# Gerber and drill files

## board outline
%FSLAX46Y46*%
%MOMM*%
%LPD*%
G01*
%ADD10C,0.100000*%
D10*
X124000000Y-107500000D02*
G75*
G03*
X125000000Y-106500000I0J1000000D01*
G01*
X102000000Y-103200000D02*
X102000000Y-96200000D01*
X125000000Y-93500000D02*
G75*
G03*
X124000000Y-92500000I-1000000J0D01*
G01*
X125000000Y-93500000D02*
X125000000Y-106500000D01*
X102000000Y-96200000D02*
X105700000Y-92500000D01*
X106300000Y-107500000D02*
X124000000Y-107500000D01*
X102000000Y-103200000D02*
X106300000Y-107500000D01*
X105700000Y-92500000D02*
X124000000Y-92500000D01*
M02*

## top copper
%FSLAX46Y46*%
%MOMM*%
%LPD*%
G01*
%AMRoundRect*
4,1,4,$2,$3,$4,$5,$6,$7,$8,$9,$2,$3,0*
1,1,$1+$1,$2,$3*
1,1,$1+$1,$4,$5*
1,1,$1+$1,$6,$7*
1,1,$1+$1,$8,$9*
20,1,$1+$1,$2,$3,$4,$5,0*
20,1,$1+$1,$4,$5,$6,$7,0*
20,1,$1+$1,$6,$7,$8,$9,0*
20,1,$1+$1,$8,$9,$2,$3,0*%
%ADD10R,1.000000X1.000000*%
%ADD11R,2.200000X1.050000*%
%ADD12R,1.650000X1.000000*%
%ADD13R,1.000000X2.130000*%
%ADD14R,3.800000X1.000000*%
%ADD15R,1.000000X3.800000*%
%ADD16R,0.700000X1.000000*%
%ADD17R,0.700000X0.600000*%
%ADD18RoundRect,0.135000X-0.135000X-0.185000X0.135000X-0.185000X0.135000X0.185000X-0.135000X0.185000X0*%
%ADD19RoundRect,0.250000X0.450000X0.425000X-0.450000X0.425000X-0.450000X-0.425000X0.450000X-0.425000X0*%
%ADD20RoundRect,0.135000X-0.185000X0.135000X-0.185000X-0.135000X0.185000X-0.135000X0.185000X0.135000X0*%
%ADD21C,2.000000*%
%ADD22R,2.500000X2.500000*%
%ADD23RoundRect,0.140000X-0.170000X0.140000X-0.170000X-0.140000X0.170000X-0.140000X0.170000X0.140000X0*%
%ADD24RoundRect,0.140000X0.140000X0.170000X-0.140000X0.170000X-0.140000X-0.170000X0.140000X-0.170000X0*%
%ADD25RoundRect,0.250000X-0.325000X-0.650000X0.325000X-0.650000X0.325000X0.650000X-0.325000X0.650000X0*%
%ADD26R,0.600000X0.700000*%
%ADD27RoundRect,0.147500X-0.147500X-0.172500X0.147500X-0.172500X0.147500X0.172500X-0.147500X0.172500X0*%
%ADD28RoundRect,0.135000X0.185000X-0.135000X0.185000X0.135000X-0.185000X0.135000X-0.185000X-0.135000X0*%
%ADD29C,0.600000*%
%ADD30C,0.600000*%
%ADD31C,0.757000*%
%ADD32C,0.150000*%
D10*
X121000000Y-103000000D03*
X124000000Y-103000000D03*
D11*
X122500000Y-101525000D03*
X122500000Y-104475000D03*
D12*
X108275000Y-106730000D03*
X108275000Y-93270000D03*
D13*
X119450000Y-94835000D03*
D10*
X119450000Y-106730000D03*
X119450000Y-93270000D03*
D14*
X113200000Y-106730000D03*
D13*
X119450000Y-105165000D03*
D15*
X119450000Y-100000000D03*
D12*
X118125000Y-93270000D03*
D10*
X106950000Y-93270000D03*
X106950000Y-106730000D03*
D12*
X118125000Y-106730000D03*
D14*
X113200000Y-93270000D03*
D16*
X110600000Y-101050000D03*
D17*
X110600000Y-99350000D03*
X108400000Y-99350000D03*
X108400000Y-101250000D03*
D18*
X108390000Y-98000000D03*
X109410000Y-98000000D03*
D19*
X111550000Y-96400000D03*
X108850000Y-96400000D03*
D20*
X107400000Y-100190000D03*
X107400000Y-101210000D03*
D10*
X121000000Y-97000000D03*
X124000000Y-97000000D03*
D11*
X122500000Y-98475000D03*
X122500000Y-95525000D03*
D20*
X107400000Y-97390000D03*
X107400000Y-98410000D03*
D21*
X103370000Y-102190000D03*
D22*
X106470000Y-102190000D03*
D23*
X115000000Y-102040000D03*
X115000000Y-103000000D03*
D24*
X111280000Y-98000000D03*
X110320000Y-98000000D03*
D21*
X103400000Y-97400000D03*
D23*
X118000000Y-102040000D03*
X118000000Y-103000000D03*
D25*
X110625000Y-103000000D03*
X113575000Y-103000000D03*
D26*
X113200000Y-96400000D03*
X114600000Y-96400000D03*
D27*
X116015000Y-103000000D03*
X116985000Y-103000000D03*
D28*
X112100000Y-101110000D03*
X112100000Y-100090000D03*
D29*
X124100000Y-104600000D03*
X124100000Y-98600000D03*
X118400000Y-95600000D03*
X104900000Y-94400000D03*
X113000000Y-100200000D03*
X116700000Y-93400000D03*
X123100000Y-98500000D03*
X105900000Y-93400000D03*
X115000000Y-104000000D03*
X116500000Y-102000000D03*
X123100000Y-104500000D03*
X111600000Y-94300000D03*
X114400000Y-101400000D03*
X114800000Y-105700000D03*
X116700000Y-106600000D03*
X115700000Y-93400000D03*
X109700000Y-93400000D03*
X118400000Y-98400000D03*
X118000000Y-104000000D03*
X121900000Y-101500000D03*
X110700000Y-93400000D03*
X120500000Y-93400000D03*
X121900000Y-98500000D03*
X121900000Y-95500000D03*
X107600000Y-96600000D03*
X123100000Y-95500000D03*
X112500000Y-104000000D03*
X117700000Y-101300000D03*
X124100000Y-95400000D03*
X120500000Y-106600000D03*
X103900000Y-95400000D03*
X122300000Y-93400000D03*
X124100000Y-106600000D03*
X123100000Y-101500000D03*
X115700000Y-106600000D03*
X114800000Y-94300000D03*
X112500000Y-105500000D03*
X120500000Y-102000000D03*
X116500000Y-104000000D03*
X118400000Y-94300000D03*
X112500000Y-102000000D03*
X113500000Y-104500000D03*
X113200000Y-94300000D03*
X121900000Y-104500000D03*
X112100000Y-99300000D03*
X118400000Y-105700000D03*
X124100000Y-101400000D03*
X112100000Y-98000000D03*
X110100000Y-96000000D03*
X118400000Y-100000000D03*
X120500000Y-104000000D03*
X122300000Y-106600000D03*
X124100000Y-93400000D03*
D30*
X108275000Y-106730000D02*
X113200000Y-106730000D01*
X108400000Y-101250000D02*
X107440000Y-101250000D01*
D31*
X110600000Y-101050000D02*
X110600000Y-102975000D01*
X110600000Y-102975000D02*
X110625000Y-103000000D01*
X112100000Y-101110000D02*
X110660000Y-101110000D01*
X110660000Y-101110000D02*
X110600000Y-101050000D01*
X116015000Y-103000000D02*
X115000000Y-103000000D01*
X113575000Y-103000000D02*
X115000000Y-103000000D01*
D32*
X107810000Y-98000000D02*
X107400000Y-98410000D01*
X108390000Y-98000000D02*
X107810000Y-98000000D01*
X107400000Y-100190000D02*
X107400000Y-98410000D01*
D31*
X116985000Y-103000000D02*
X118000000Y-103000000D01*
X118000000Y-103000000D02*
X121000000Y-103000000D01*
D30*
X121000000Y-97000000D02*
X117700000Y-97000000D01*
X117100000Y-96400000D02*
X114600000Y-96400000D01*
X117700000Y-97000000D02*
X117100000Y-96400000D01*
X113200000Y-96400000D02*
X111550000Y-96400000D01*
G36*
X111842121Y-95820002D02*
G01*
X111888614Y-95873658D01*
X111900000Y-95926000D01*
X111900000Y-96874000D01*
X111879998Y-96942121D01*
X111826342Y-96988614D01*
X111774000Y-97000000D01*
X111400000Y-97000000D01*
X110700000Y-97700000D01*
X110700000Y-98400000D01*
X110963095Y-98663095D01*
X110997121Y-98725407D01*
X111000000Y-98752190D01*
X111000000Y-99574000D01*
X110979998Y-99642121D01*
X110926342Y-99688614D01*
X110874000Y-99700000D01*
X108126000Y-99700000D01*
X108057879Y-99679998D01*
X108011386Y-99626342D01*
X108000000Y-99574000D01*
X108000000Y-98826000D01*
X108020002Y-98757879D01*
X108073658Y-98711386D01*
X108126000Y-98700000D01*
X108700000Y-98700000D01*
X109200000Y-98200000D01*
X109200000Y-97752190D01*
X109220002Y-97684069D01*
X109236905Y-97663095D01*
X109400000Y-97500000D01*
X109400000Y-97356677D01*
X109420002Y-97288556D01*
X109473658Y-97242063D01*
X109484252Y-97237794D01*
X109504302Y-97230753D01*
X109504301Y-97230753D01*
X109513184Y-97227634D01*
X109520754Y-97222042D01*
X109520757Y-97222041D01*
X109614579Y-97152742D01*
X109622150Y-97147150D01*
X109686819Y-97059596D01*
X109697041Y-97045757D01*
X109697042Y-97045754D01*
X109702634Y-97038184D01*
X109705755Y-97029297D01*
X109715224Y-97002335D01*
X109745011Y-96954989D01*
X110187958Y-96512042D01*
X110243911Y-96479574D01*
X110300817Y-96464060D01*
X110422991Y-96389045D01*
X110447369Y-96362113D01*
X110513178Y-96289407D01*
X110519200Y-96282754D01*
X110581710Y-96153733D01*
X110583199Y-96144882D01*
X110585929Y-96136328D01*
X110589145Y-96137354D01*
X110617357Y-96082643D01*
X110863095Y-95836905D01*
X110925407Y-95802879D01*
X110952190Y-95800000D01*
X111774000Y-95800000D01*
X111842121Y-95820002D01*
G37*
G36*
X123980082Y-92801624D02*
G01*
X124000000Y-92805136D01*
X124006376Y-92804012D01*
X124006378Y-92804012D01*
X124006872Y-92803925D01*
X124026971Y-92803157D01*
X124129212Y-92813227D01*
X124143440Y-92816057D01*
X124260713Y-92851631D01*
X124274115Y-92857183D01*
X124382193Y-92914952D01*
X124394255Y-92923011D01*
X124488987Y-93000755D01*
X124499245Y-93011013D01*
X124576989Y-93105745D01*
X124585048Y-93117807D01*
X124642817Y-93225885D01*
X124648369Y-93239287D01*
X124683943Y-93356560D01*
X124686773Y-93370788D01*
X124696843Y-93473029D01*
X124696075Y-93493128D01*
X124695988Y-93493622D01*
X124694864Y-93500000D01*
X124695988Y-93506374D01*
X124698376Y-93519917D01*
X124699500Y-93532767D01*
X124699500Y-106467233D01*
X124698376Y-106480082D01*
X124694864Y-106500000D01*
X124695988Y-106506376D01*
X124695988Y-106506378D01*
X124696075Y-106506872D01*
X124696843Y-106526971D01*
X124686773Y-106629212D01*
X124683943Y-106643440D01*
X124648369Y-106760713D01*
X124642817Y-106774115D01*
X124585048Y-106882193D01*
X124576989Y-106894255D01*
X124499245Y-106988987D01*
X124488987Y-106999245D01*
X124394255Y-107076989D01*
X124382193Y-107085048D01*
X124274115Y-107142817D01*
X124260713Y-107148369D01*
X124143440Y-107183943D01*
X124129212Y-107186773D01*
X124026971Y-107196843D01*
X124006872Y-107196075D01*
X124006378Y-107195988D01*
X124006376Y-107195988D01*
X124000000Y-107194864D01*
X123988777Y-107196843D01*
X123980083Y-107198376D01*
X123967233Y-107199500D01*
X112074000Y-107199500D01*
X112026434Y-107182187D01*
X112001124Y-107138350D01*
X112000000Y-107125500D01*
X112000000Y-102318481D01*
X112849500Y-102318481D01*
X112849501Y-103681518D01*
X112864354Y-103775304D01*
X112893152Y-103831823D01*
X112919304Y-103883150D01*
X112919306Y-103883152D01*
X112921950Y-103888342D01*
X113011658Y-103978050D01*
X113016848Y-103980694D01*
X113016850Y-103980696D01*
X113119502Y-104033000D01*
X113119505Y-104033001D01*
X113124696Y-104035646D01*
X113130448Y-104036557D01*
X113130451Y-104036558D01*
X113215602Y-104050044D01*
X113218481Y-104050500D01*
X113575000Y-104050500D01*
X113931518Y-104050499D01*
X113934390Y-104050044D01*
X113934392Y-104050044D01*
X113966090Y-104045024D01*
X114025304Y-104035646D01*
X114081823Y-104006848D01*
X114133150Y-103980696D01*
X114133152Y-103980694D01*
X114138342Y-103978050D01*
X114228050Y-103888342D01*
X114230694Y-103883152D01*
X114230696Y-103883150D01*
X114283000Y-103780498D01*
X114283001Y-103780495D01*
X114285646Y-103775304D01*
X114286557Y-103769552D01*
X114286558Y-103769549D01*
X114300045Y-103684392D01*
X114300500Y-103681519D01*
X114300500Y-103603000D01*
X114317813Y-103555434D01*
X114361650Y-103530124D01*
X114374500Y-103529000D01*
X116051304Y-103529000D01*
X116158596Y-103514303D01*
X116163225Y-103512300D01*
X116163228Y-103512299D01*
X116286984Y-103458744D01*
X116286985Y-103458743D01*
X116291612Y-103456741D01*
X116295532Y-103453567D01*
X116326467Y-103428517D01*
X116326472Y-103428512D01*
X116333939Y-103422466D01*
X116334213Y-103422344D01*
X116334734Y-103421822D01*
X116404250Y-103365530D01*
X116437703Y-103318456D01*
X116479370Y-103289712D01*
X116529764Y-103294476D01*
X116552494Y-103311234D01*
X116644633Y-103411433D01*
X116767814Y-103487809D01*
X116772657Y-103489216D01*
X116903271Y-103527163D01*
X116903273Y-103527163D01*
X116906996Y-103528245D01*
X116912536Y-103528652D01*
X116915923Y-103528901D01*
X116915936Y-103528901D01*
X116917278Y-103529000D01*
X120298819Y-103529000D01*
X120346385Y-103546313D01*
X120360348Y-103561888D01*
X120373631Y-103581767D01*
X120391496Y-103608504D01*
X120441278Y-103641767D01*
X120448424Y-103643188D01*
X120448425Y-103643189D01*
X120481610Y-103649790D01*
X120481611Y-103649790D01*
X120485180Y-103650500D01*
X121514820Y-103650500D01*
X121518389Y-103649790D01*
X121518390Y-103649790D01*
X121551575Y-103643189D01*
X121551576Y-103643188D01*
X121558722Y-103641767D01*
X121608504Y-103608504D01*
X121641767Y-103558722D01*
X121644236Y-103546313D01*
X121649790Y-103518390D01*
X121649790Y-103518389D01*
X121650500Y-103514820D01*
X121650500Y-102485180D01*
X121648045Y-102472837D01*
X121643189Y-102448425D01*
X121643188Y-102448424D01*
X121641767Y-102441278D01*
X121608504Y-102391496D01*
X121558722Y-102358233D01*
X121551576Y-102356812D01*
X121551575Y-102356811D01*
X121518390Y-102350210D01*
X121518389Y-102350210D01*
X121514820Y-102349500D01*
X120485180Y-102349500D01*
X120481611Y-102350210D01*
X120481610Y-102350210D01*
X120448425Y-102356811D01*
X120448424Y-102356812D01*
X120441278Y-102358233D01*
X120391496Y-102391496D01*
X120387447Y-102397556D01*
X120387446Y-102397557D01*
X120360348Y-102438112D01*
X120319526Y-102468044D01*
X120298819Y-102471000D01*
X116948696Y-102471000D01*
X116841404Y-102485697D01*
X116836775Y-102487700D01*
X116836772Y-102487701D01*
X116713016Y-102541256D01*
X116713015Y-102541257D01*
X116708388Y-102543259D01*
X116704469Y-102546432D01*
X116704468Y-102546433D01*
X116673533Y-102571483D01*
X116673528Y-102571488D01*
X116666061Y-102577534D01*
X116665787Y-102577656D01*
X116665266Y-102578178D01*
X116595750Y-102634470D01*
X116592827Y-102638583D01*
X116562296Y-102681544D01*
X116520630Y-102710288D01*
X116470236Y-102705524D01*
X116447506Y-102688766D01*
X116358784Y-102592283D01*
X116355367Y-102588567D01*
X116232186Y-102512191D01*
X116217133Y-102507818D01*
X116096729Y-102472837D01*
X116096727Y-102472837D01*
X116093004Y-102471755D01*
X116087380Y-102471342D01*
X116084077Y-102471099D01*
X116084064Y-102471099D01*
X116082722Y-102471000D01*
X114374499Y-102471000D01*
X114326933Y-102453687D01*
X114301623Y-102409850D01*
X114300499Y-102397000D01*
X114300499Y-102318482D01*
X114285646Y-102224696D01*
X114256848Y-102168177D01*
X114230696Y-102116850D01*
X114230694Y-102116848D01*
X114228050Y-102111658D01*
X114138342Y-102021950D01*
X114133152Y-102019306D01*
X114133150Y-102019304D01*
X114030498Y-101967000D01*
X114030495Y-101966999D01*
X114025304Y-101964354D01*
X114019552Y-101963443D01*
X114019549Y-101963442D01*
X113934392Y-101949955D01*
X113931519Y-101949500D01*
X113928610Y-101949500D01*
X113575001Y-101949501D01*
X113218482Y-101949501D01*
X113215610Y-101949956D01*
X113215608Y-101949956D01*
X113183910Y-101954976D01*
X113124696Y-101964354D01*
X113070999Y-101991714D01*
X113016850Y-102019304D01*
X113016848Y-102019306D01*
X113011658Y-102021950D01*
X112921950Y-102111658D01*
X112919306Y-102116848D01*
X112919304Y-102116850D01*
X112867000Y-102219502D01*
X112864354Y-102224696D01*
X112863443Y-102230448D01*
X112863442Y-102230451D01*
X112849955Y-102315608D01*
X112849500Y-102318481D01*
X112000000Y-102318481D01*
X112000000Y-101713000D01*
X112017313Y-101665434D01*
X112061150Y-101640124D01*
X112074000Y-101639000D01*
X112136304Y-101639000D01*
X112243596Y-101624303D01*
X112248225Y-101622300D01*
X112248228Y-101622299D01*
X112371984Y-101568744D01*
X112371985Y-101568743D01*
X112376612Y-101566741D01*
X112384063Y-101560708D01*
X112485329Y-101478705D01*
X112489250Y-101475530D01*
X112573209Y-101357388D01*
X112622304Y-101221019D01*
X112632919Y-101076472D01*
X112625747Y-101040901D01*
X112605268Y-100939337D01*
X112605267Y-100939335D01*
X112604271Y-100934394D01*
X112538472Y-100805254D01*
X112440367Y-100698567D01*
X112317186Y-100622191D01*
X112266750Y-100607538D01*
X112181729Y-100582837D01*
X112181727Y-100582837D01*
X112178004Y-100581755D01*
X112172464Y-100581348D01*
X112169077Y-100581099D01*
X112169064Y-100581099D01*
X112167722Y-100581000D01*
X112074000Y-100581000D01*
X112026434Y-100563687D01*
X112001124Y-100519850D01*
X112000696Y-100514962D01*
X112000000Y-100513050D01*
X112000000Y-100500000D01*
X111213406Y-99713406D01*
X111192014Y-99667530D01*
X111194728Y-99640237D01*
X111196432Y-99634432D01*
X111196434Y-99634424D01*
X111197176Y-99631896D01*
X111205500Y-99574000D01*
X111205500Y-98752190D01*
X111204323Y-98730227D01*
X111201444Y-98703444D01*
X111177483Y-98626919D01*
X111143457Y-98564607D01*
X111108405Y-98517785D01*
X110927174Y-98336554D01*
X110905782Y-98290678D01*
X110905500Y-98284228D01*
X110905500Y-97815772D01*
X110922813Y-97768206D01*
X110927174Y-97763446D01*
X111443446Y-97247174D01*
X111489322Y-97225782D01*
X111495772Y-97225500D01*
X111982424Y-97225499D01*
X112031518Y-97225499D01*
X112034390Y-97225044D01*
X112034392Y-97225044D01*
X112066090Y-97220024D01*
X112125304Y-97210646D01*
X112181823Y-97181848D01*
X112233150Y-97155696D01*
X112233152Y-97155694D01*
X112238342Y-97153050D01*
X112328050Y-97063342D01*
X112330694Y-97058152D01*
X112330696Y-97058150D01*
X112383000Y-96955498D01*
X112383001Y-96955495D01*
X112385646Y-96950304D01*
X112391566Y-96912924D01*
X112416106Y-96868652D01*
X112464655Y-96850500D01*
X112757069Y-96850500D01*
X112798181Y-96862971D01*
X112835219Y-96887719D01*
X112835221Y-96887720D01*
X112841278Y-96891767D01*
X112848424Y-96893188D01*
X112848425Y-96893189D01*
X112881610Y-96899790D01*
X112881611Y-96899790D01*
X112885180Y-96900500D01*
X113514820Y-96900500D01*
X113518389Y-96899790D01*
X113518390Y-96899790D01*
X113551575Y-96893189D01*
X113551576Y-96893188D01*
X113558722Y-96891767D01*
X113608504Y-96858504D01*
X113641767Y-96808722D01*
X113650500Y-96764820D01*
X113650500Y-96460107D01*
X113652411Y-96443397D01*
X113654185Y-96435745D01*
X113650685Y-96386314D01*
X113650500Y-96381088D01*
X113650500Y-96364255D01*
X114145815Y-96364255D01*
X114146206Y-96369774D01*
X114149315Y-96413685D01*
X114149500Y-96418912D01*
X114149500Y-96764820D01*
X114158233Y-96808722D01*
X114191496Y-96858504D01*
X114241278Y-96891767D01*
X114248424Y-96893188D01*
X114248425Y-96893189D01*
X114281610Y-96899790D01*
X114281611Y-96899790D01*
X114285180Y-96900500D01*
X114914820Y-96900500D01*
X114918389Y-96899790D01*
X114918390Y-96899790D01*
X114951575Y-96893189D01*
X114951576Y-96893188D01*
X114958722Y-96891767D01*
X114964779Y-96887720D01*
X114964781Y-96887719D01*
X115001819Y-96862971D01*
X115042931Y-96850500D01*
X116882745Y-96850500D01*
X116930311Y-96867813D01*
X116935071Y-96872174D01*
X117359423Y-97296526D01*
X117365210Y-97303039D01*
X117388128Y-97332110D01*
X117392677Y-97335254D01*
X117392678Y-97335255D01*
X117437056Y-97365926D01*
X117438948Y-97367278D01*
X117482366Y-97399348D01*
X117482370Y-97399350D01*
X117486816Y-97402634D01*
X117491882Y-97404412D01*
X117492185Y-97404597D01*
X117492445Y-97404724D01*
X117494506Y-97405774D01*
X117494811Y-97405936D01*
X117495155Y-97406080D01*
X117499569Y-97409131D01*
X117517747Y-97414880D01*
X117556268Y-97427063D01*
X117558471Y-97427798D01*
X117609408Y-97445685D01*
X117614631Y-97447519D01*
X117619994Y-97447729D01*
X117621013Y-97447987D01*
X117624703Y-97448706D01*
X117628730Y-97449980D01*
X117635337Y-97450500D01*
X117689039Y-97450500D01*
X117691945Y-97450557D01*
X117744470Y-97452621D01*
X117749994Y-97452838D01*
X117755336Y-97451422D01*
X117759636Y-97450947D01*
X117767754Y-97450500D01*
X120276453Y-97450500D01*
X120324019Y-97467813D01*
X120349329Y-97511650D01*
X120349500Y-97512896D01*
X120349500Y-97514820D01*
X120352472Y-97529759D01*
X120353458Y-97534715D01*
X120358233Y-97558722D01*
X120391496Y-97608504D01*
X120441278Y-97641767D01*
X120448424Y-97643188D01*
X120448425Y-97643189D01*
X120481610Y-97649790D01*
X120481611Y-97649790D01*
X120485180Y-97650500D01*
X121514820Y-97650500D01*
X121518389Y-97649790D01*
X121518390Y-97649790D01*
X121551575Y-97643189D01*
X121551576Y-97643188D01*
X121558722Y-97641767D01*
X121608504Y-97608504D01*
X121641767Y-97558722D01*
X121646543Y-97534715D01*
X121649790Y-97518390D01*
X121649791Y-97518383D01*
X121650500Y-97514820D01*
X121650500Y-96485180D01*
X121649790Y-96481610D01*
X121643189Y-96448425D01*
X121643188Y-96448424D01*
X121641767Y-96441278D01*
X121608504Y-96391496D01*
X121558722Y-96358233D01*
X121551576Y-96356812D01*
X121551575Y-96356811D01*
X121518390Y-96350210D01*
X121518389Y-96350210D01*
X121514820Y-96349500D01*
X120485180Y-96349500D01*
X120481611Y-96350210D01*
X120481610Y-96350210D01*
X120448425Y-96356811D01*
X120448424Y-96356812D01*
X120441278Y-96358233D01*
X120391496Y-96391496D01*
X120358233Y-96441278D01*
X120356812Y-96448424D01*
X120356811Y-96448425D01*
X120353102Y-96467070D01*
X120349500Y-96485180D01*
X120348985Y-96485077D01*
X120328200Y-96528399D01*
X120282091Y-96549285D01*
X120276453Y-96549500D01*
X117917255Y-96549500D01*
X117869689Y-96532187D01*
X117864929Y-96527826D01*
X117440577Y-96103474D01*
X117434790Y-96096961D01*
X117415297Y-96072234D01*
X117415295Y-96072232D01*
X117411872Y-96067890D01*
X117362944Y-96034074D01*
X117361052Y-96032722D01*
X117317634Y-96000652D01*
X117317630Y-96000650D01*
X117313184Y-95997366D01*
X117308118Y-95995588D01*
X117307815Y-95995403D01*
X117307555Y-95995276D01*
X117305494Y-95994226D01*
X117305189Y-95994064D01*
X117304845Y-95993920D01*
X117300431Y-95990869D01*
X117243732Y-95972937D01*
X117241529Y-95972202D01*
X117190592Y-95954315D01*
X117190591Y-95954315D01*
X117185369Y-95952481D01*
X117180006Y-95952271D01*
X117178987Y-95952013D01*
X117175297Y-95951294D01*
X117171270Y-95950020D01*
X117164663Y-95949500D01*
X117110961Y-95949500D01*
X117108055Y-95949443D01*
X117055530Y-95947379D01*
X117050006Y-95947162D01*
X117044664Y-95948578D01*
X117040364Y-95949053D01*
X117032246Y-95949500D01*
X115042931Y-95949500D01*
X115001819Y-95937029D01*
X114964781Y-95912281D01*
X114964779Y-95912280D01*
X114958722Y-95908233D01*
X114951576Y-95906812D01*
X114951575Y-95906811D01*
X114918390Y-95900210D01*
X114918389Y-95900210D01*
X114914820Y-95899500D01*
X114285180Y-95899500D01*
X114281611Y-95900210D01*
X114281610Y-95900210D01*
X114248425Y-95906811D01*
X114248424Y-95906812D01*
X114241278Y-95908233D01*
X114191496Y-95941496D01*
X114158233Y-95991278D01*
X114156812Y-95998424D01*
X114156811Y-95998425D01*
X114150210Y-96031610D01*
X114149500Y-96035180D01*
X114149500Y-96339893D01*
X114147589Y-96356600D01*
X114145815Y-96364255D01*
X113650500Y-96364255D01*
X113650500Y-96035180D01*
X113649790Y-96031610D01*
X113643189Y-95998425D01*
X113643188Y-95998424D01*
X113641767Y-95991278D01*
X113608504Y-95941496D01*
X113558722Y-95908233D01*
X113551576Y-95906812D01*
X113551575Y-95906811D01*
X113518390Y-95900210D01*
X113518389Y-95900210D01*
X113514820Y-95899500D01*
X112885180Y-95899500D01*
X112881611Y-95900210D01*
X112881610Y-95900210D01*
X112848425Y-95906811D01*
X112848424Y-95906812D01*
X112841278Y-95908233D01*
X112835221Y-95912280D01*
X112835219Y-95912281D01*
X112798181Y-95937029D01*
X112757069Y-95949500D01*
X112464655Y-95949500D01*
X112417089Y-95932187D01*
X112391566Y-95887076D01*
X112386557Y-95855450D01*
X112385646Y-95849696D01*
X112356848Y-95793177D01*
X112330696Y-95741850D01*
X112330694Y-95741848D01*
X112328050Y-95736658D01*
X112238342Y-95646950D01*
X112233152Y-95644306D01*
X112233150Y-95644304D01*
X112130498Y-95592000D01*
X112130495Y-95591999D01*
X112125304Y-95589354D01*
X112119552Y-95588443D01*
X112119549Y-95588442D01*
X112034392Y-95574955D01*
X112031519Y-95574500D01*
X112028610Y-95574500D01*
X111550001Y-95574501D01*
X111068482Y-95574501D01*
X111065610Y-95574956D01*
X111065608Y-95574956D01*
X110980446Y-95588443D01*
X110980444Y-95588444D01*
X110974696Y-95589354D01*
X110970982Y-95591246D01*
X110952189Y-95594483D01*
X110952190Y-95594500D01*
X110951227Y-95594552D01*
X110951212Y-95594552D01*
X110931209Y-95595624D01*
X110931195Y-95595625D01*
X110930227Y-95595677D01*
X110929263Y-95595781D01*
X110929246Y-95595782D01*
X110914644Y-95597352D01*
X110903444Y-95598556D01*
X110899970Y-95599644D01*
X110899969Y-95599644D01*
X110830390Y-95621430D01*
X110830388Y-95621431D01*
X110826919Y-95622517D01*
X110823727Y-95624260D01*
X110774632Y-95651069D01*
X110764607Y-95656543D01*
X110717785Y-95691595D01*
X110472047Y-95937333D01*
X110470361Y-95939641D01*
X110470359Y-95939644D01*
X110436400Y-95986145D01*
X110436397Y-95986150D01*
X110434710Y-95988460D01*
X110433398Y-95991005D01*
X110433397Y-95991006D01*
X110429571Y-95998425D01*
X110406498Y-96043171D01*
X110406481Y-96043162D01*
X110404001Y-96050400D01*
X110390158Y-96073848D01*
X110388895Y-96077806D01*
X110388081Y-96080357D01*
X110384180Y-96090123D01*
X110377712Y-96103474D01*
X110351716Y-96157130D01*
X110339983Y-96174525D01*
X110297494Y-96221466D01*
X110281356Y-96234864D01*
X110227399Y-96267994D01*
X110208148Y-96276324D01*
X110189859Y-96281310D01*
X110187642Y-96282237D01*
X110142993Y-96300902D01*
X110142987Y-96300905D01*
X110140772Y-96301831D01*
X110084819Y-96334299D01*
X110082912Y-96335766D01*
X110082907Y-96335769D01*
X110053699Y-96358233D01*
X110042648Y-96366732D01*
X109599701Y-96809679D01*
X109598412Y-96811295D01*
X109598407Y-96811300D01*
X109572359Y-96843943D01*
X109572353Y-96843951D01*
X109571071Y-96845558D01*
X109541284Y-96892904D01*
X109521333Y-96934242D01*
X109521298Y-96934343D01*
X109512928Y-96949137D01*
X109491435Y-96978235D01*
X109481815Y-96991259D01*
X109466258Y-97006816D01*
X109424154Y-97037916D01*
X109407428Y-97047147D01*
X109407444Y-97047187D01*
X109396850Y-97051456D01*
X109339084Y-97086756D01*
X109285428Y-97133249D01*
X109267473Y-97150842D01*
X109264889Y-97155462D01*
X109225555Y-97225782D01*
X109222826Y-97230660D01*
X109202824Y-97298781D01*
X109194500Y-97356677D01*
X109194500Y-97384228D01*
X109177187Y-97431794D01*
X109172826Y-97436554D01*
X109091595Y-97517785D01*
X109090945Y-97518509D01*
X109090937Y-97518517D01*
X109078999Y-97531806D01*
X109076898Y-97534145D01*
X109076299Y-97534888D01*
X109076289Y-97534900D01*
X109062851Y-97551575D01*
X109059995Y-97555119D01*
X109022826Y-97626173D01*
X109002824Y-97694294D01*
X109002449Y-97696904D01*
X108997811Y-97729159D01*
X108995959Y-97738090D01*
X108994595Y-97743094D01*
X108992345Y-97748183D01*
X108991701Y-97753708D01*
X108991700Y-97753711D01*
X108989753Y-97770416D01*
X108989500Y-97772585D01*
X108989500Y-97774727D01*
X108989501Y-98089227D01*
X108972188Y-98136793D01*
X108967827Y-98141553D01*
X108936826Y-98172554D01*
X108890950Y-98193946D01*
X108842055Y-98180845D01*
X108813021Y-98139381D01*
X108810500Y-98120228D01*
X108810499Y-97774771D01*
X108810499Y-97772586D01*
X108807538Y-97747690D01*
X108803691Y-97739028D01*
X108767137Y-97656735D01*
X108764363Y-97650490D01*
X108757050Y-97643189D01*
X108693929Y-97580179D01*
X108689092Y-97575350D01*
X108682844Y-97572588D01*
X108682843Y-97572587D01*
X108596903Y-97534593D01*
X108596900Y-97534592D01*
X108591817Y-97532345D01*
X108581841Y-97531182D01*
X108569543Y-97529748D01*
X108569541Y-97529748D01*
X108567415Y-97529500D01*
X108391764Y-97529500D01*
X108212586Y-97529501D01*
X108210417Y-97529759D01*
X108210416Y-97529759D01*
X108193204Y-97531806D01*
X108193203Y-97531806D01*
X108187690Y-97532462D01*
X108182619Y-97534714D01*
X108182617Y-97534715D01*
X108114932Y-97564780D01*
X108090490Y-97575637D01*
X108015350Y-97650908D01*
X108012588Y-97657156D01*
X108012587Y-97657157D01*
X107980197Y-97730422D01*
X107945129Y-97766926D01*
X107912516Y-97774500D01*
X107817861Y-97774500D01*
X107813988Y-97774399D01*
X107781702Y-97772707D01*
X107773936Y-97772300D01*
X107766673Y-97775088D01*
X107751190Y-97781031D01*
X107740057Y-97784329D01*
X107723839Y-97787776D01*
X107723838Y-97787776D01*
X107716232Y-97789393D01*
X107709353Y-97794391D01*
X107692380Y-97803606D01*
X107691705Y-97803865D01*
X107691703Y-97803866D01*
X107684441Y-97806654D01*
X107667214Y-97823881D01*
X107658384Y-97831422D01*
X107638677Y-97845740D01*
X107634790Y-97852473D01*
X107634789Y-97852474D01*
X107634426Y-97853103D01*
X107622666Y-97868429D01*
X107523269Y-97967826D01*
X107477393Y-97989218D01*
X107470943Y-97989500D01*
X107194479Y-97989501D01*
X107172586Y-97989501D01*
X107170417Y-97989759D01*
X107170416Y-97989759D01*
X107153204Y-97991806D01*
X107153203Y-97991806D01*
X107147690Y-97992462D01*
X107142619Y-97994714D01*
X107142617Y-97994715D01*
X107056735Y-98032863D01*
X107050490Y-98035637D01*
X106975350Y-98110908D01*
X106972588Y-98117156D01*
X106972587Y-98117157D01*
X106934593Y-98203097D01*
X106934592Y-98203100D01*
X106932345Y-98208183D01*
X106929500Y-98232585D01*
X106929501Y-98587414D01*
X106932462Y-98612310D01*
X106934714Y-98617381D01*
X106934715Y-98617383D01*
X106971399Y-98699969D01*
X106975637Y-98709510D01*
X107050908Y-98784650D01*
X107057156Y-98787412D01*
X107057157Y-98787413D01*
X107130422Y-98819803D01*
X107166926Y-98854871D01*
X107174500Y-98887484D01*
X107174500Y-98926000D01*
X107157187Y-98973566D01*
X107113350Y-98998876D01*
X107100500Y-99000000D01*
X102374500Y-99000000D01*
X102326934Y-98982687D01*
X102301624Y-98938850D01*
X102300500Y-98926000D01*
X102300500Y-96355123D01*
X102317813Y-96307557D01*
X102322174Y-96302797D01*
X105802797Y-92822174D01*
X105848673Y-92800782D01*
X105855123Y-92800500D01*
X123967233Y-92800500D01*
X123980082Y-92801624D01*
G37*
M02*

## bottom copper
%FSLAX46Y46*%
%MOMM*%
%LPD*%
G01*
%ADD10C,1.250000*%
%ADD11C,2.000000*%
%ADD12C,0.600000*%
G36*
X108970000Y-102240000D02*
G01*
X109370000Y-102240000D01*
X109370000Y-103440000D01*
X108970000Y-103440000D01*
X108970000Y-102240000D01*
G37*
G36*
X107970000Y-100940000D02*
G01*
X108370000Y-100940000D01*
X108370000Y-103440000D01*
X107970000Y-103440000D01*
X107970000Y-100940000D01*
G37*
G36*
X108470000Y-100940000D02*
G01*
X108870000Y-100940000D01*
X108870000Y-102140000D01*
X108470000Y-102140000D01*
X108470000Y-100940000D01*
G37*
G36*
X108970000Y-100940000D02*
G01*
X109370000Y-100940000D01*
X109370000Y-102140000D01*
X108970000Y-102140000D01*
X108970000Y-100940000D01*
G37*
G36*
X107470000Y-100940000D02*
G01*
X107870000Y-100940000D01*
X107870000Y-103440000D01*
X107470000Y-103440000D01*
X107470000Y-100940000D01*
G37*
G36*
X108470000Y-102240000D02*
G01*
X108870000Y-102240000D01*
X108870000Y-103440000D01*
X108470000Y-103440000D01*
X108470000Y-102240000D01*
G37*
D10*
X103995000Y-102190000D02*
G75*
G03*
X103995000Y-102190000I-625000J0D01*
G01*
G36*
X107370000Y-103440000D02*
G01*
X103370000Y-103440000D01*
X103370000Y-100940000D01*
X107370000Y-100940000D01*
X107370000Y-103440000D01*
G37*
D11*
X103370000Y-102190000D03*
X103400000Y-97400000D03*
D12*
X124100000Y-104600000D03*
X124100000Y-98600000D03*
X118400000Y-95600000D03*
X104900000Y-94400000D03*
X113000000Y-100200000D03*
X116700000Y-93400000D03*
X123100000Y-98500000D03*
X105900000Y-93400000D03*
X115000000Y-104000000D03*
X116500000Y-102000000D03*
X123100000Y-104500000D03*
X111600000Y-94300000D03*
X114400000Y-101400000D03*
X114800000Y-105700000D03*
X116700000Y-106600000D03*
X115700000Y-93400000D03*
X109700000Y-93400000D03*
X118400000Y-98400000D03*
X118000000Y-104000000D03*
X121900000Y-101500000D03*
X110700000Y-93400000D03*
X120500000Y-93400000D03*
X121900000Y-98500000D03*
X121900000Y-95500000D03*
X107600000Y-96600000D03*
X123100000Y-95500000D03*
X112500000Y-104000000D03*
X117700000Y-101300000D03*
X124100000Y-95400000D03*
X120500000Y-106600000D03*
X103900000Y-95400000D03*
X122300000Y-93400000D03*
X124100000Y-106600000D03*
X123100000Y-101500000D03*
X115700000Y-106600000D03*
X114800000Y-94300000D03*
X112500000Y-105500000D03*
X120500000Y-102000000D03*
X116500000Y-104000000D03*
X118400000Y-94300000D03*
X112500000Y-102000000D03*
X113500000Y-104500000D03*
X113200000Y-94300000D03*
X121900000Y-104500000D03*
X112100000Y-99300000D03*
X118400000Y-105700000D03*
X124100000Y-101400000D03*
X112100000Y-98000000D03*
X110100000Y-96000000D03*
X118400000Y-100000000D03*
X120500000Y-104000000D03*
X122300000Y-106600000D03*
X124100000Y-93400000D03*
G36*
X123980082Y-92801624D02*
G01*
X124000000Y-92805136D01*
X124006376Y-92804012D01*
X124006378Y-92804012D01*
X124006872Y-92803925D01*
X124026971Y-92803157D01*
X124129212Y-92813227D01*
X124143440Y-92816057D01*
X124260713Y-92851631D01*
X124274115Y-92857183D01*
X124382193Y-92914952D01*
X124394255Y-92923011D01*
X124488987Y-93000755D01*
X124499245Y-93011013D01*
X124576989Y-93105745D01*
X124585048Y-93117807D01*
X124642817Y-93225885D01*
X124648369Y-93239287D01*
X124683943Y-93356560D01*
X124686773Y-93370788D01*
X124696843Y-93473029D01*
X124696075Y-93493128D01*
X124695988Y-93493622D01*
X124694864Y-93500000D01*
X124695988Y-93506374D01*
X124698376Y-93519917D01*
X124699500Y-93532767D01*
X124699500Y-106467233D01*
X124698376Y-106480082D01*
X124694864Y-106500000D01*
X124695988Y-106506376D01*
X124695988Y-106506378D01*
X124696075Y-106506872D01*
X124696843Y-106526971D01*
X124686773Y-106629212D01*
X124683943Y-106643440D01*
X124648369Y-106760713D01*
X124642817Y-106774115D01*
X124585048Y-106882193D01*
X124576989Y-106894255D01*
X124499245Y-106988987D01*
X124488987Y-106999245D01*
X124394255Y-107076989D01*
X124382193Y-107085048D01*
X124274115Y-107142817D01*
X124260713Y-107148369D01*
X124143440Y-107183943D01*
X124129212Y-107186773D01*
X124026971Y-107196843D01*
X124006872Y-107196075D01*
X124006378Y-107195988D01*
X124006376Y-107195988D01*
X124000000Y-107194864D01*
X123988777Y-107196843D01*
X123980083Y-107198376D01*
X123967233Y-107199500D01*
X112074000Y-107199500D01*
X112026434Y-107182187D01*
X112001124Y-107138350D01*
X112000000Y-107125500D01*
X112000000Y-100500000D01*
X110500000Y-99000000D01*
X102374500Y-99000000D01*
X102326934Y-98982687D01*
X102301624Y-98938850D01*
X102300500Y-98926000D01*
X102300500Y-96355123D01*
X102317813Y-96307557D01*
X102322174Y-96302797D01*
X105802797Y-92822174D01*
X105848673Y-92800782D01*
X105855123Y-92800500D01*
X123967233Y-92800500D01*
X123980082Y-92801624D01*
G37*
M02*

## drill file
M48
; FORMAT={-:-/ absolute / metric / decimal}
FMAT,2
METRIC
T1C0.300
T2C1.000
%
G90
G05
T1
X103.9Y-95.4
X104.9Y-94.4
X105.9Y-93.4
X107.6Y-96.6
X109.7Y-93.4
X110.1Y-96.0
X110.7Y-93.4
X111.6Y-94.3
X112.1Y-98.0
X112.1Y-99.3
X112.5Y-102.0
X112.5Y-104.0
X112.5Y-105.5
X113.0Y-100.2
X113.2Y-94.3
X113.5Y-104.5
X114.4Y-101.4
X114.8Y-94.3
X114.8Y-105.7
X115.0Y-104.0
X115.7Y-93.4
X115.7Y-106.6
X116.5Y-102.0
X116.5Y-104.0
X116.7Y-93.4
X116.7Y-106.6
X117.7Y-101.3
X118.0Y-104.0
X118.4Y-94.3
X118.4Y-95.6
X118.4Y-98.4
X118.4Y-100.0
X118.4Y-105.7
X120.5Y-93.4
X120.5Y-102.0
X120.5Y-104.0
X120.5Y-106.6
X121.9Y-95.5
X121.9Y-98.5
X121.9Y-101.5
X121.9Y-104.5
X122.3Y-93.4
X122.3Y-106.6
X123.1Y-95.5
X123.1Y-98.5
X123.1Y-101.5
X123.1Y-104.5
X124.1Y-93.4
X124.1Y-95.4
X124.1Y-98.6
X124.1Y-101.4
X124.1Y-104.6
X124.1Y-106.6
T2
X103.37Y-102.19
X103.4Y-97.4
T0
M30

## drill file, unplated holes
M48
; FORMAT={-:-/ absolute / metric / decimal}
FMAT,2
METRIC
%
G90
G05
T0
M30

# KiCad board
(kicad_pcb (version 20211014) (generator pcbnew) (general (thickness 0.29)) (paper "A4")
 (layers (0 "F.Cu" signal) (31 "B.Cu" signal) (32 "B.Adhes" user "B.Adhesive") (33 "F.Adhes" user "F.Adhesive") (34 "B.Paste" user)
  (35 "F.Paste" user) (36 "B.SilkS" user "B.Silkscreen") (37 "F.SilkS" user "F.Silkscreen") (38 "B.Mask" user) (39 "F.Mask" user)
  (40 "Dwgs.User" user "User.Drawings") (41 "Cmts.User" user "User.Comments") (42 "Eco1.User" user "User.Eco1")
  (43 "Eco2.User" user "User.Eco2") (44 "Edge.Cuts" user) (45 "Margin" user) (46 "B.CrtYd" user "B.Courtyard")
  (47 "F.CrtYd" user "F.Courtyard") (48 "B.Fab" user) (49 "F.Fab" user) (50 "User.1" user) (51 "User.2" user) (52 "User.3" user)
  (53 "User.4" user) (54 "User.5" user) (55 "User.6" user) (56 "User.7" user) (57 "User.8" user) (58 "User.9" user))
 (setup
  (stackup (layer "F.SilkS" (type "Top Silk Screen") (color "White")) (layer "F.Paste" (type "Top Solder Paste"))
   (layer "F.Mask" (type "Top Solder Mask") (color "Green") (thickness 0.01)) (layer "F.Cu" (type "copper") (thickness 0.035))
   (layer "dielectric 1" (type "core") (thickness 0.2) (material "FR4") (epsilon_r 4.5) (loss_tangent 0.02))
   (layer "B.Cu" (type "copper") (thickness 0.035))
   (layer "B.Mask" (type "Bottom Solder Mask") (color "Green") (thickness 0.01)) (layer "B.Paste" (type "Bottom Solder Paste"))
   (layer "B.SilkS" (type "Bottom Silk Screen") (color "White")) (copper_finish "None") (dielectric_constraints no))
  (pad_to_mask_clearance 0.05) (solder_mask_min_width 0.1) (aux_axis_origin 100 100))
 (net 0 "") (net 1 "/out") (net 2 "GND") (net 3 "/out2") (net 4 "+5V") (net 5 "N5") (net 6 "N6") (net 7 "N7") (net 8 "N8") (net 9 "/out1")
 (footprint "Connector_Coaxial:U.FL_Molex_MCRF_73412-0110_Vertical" (layer "F.Cu") (at 122.5 103 -90)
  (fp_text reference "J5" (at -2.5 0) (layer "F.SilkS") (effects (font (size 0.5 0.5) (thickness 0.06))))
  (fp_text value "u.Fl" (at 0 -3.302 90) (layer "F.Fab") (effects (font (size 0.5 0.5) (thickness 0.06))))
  (pad "1" smd rect (at 0 1.5 270) (size 1 1) (layers "F.Cu" "F.Paste" "F.Mask") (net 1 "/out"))
  (pad "2" smd rect (at 0 -1.5 270) (size 1 1) (layers "F.Cu" "F.Paste" "F.Mask") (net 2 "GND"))
  (pad "2" smd rect (at -1.475 0 270) (size 1.05 2.2) (layers "F.Cu" "F.Paste" "F.Mask") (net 2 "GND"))
  (pad "2" smd rect (at 1.475 0 270) (size 1.05 2.2) (layers "F.Cu" "F.Paste" "F.Mask") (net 2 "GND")))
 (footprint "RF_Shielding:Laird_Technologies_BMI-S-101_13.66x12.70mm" (layer "F.Cu") (at 113.2 100) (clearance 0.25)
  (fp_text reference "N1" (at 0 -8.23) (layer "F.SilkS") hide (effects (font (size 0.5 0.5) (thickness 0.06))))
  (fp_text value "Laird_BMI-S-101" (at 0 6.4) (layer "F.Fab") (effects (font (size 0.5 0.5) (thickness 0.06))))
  (pad "1" smd rect (at -4.925 6.73) (size 1.65 1) (layers "F.Cu" "F.Paste" "F.Mask") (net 2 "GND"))
  (pad "1" smd rect (at -4.925 -6.73) (size 1.65 1) (layers "F.Cu" "F.Paste" "F.Mask") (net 2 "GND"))
  (pad "1" smd rect (at 6.25 -5.165) (size 1 2.13) (layers "F.Cu" "F.Paste" "F.Mask") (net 2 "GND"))
  (pad "1" smd rect (at 6.25 6.73) (size 1 1) (layers "F.Cu" "F.Paste" "F.Mask") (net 2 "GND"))
  (pad "1" smd rect (at 6.25 -6.73) (size 1 1) (layers "F.Cu" "F.Paste" "F.Mask") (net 2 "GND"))
  (pad "1" smd rect (at 0 6.73) (size 3.8 1) (layers "F.Cu" "F.Paste" "F.Mask") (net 2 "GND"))
  (pad "1" smd rect (at 6.25 5.165) (size 1 2.13) (layers "F.Cu" "F.Paste" "F.Mask") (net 2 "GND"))
  (pad "1" smd rect (at 6.25 0) (size 1 3.8) (layers "F.Cu" "F.Paste" "F.Mask") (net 2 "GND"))
  (pad "1" smd rect (at 4.925 -6.73) (size 1.65 1) (layers "F.Cu" "F.Paste" "F.Mask") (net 2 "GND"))
  (pad "1" smd rect (at -6.25 -6.73) (size 1 1) (layers "F.Cu" "F.Paste" "F.Mask") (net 2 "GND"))
  (pad "1" smd rect (at -6.25 6.73) (size 1 1) (layers "F.Cu" "F.Paste" "F.Mask") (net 2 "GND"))
  (pad "1" smd rect (at 4.925 6.73) (size 1.65 1) (layers "F.Cu" "F.Paste" "F.Mask") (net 2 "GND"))
  (pad "1" smd rect (at 0 -6.73) (size 3.8 1) (layers "F.Cu" "F.Paste" "F.Mask") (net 2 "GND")))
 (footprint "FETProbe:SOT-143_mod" (layer "F.Cu") (at 109.5 100.3 180)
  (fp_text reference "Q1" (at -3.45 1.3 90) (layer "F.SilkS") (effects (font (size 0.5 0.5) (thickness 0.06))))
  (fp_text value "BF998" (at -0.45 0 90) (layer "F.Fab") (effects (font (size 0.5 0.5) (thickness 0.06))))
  (pad "1" smd rect (at -1.1 -0.75 180) (size 0.7 1) (layers "F.Cu" "F.Paste" "F.Mask") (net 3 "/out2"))
  (pad "2" smd rect (at -1.1 0.95 180) (size 0.7 0.6) (layers "F.Cu" "F.Paste" "F.Mask") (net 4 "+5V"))
  (pad "3" smd rect (at 1.1 0.95 180) (size 0.7 0.6) (layers "F.Cu" "F.Paste" "F.Mask") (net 4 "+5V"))
  (pad "4" smd rect (at 1.1 -0.95 180) (size 0.7 0.6) (layers "F.Cu" "F.Paste" "F.Mask") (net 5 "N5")))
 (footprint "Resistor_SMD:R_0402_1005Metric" (layer "F.Cu") (at 108.9 98)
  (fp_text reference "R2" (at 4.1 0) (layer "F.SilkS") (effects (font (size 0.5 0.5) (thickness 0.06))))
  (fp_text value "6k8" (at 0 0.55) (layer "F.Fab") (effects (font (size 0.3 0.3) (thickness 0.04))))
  (pad "1" smd roundrect (at -0.51 0) (size 0.54 0.64) (layers "F.Cu" "F.Paste" "F.Mask") (roundrect_rratio 0.25) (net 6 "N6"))
  (pad "2" smd roundrect (at 0.51 0) (size 0.54 0.64) (layers "F.Cu" "F.Paste" "F.Mask") (roundrect_rratio 0.25) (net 4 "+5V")))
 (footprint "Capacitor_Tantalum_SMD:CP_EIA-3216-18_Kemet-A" (layer "F.Cu") (at 110.2 96.4 180)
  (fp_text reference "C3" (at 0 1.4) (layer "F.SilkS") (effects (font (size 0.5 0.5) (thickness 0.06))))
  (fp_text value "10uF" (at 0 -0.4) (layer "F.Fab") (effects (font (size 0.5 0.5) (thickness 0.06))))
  (pad "1" smd roundrect (at -1.35 0 180) (size 1.4 1.35) (layers "F.Cu" "F.Paste" "F.Mask") (roundrect_rratio 0.1851851852) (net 4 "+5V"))
  (pad "2" smd roundrect (at 1.35 0 180) (size 1.4 1.35) (layers "F.Cu" "F.Paste" "F.Mask") (roundrect_rratio 0.1851851852) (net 2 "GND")))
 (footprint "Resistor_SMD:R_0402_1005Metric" (layer "F.Cu") (at 107.4 100.7 -90)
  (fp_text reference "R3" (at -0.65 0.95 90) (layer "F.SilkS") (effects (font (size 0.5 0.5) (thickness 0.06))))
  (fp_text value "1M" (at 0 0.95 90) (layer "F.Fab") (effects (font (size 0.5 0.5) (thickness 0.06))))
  (pad "1" smd roundrect (at -0.51 0 270) (size 0.54 0.64) (layers "F.Cu" "F.Paste" "F.Mask") (roundrect_rratio 0.25) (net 6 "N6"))
  (pad "2" smd roundrect (at 0.51 0 270) (size 0.54 0.64) (layers "F.Cu" "F.Paste" "F.Mask") (roundrect_rratio 0.25) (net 5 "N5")))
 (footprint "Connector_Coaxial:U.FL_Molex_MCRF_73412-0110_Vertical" (layer "F.Cu") (at 122.5 97 -90)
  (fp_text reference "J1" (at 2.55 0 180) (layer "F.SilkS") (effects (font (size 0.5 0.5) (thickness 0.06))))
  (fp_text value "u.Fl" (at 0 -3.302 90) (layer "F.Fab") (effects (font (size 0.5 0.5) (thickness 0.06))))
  (pad "1" smd rect (at 0 1.5 270) (size 1 1) (layers "F.Cu" "F.Paste" "F.Mask") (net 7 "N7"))
  (pad "2" smd rect (at 0 -1.5 270) (size 1 1) (layers "F.Cu" "F.Paste" "F.Mask") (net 2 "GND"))
  (pad "2" smd rect (at 1.475 0 270) (size 1.05 2.2) (layers "F.Cu" "F.Paste" "F.Mask") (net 2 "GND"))
  (pad "2" smd rect (at -1.475 0 270) (size 1.05 2.2) (layers "F.Cu" "F.Paste" "F.Mask") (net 2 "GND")))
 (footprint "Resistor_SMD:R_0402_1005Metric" (layer "F.Cu") (at 107.4 97.9 -90)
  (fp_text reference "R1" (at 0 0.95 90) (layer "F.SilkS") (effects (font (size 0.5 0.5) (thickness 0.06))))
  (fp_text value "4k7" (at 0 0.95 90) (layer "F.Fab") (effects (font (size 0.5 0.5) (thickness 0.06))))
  (pad "1" smd roundrect (at -0.51 0 270) (size 0.54 0.64) (layers "F.Cu" "F.Paste" "F.Mask") (roundrect_rratio 0.25) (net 2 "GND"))
  (pad "2" smd roundrect (at 0.51 0 270) (size 0.54 0.64) (layers "F.Cu" "F.Paste" "F.Mask") (roundrect_rratio 0.25) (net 6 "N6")))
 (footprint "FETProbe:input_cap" (layer "F.Cu") (at 108.07 102.19)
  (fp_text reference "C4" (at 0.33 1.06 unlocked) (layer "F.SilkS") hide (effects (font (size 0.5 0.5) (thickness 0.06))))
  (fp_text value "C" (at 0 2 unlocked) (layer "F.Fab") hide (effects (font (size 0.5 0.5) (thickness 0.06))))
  (fp_rect (start 0.9 0.05) (end 1.3 1.25) (layer "B.Cu") (width 0) (fill solid))
  (fp_rect (start -0.1 -1.25) (end 0.3 1.25) (layer "B.Cu") (width 0) (fill solid))
  (fp_rect (start 0.4 -1.25) (end 0.8 -0.05) (layer "B.Cu") (width 0) (fill solid))
  (fp_rect (start 0.9 -1.25) (end 1.3 -0.05) (layer "B.Cu") (width 0) (fill solid))
  (fp_rect (start -0.6 -1.25) (end -0.2 1.25) (layer "B.Cu") (width 0) (fill solid))
  (fp_rect (start 0.4 0.05) (end 0.8 1.25) (layer "B.Cu") (width 0) (fill solid))
  (fp_circle (center -4.7 0) (end -3.45 0) (layer "B.Cu") (width 0) (fill solid))
  (fp_poly (pts (xy -4.7 -1.25) (xy -0.7 -1.25) (xy -0.7 1.25) (xy -4.7 1.25)) (layer "B.Cu") (width 0) (fill solid))
  (pad "1" thru_hole circle (at -4.7 0) (size 2 2) (drill 1) (layers *.Cu *.Mask) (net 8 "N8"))
  (pad "2" smd rect (at -1.6 0) (size 2.5 2.5) (layers "F.Cu") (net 5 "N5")))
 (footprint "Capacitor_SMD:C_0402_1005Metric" (layer "F.Cu") (at 115 102.52 -90)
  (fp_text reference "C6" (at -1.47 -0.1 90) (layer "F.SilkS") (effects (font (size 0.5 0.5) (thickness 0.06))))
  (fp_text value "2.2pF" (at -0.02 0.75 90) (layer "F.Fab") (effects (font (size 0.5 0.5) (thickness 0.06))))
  (pad "1" smd roundrect (at -0.48 0 270) (size 0.56 0.62) (layers "F.Cu" "F.Paste" "F.Mask") (roundrect_rratio 0.25) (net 2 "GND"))
  (pad "2" smd roundrect (at 0.48 0 270) (size 0.56 0.62) (layers "F.Cu" "F.Paste" "F.Mask") (roundrect_rratio 0.25) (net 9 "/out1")))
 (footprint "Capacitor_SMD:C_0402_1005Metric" (layer "F.Cu") (at 110.8 98 180)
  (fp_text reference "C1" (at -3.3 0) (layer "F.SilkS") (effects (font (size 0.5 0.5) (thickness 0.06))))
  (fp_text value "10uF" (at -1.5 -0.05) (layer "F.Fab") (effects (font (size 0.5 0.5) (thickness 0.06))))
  (pad "1" smd roundrect (at -0.48 0 180) (size 0.56 0.62) (layers "F.Cu" "F.Paste" "F.Mask") (roundrect_rratio 0.25) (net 2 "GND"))
  (pad "2" smd roundrect (at 0.48 0 180) (size 0.56 0.62) (layers "F.Cu" "F.Paste" "F.Mask") (roundrect_rratio 0.25) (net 4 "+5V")))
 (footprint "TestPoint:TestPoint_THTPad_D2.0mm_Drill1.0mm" (layer "F.Cu") (at 103.4 97.4)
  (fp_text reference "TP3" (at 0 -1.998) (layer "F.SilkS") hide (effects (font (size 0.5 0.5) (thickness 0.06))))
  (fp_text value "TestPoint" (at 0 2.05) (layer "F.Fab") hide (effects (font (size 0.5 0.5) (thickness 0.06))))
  (pad "1" thru_hole circle (at 0 0) (size 2 2) (drill 1) (layers *.Cu *.Mask) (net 2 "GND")))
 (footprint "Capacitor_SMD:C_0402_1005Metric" (layer "F.Cu") (at 118 102.52 -90)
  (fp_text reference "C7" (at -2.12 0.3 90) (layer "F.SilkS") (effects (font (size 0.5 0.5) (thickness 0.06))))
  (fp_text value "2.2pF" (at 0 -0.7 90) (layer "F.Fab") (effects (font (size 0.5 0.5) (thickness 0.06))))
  (pad "1" smd roundrect (at -0.48 0 270) (size 0.56 0.62) (layers "F.Cu" "F.Paste" "F.Mask") (roundrect_rratio 0.25) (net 2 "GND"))
  (pad "2" smd roundrect (at 0.48 0 270) (size 0.56 0.62) (layers "F.Cu" "F.Paste" "F.Mask") (roundrect_rratio 0.25) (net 1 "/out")))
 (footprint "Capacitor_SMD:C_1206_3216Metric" (layer "F.Cu") (at 112.1 103)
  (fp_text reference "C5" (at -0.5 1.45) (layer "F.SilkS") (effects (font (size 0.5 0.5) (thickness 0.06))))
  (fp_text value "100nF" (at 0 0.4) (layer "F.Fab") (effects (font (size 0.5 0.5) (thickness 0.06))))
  (pad "1" smd roundrect (at -1.475 0) (size 1.15 1.8) (layers "F.Cu" "F.Paste" "F.Mask") (roundrect_rratio 0.2173913043) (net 3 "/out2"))
  (pad "2" smd roundrect (at 1.475 0) (size 1.15 1.8) (layers "F.Cu" "F.Paste" "F.Mask") (roundrect_rratio 0.2173913043) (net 9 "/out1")))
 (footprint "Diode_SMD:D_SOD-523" (layer "F.Cu") (at 113.9 96.4)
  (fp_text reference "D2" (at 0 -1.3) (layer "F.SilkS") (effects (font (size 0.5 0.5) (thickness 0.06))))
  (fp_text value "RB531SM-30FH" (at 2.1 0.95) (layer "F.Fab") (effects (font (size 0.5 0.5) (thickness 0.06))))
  (pad "1" smd rect (at -0.7 0 180) (size 0.6 0.7) (layers "F.Cu" "F.Paste" "F.Mask") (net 4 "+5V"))
  (pad "2" smd rect (at 0.7 0 180) (size 0.6 0.7) (layers "F.Cu" "F.Paste" "F.Mask") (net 7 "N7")))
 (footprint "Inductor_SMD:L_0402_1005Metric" (layer "F.Cu") (at 116.5 103)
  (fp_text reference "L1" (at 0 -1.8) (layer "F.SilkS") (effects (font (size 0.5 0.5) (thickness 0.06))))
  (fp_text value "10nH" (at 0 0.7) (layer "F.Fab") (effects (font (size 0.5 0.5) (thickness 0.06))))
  (pad "1" smd roundrect (at -0.485 0) (size 0.59 0.64) (layers "F.Cu" "F.Paste" "F.Mask") (roundrect_rratio 0.25) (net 9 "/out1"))
  (pad "2" smd roundrect (at 0.485 0) (size 0.59 0.64) (layers "F.Cu" "F.Paste" "F.Mask") (roundrect_rratio 0.25) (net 1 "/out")))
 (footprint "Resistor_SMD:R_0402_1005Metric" (layer "F.Cu") (at 112.1 100.6 90)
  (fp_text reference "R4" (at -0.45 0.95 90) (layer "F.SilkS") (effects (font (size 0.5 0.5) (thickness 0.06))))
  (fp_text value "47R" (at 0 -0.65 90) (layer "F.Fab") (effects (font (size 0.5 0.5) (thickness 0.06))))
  (pad "1" smd roundrect (at -0.51 0 90) (size 0.54 0.64) (layers "F.Cu" "F.Paste" "F.Mask") (roundrect_rratio 0.25) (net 3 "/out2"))
  (pad "2" smd roundrect (at 0.51 0 90) (size 0.54 0.64) (layers "F.Cu" "F.Paste" "F.Mask") (roundrect_rratio 0.25) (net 2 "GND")))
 (gr_arc (start 125 106.5) (mid 124.707107 107.207107) (end 124 107.5) (layer "Edge.Cuts") (width 0.1))
 (gr_line (start 102 103.2) (end 102 96.2) (layer "Edge.Cuts") (width 0.1))
 (gr_arc (start 124 92.5) (mid 124.707107 92.792893) (end 125 93.5) (layer "Edge.Cuts") (width 0.1))
 (gr_line (start 125 93.5) (end 125 106.5) (layer "Edge.Cuts") (width 0.1))
 (gr_line (start 102 96.2) (end 105.7 92.5) (layer "Edge.Cuts") (width 0.1))
 (gr_line (start 106.3 107.5) (end 124 107.5) (layer "Edge.Cuts") (width 0.1))
 (gr_line (start 102 103.2) (end 106.3 107.5) (layer "Edge.Cuts") (width 0.1))
 (gr_line (start 105.7 92.5) (end 124 92.5) (layer "Edge.Cuts") (width 0.1))
 (segment (start 108.275 106.73) (end 113.2 106.73) (width 0.6) (layer "F.Cu") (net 2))
 (via (at 124.1 104.6) (size 0.6) (drill 0.3) (layers "F.Cu" "B.Cu") (free) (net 2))
 (via (at 124.1 98.6) (size 0.6) (drill 0.3) (layers "F.Cu" "B.Cu") (free) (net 2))
 (via (at 118.4 95.6) (size 0.6) (drill 0.3) (layers "F.Cu" "B.Cu") (free) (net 2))
 (via (at 104.9 94.4) (size 0.6) (drill 0.3) (layers "F.Cu" "B.Cu") (free) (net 2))
 (via (at 113 100.2) (size 0.6) (drill 0.3) (layers "F.Cu" "B.Cu") (free) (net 2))
 (via (at 116.7 93.4) (size 0.6) (drill 0.3) (layers "F.Cu" "B.Cu") (free) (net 2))
 (via (at 123.1 98.5) (size 0.6) (drill 0.3) (layers "F.Cu" "B.Cu") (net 2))
 (via (at 105.9 93.4) (size 0.6) (drill 0.3) (layers "F.Cu" "B.Cu") (free) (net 2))
 (via (at 115 104) (size 0.6) (drill 0.3) (layers "F.Cu" "B.Cu") (free) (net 2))
 (via (at 116.5 102) (size 0.6) (drill 0.3) (layers "F.Cu" "B.Cu") (free) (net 2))
 (via (at 123.1 104.5) (size 0.6) (drill 0.3) (layers "F.Cu" "B.Cu") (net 2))
 (via (at 111.6 94.3) (size 0.6) (drill 0.3) (layers "F.Cu" "B.Cu") (free) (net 2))
 (via (at 114.4 101.4) (size 0.6) (drill 0.3) (layers "F.Cu" "B.Cu") (free) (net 2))
 (via (at 114.8 105.7) (size 0.6) (drill 0.3) (layers "F.Cu" "B.Cu") (free) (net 2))
 (via (at 116.7 106.6) (size 0.6) (drill 0.3) (layers "F.Cu" "B.Cu") (free) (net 2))
 (via (at 115.7 93.4) (size 0.6) (drill 0.3) (layers "F.Cu" "B.Cu") (free) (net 2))
 (via (at 109.7 93.4) (size 0.6) (drill 0.3) (layers "F.Cu" "B.Cu") (free) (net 2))
 (via (at 118.4 98.4) (size 0.6) (drill 0.3) (layers "F.Cu" "B.Cu") (free) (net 2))
 (via (at 118 104) (size 0.6) (drill 0.3) (layers "F.Cu" "B.Cu") (free) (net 2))
 (via (at 121.9 101.5) (size 0.6) (drill 0.3) (layers "F.Cu" "B.Cu") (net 2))
 (via (at 110.7 93.4) (size 0.6) (drill 0.3) (layers "F.Cu" "B.Cu") (free) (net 2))
 (via (at 120.5 93.4) (size 0.6) (drill 0.3) (layers "F.Cu" "B.Cu") (free) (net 2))
 (via (at 121.9 98.5) (size 0.6) (drill 0.3) (layers "F.Cu" "B.Cu") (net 2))
 (via (at 121.9 95.5) (size 0.6) (drill 0.3) (layers "F.Cu" "B.Cu") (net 2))
 (via (at 107.6 96.6) (size 0.6) (drill 0.3) (layers "F.Cu" "B.Cu") (free) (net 2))
 (via (at 123.1 95.5) (size 0.6) (drill 0.3) (layers "F.Cu" "B.Cu") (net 2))
 (via (at 112.5 104) (size 0.6) (drill 0.3) (layers "F.Cu" "B.Cu") (free) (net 2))
 (via (at 117.7 101.3) (size 0.6) (drill 0.3) (layers "F.Cu" "B.Cu") (free) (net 2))
 (via (at 124.1 95.4) (size 0.6) (drill 0.3) (layers "F.Cu" "B.Cu") (free) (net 2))
 (via (at 120.5 106.6) (size 0.6) (drill 0.3) (layers "F.Cu" "B.Cu") (free) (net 2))
 (via (at 103.9 95.4) (size 0.6) (drill 0.3) (layers "F.Cu" "B.Cu") (free) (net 2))
 (via (at 122.3 93.4) (size 0.6) (drill 0.3) (layers "F.Cu" "B.Cu") (free) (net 2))
 (via (at 124.1 106.6) (size 0.6) (drill 0.3) (layers "F.Cu" "B.Cu") (free) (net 2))
 (via (at 123.1 101.5) (size 0.6) (drill 0.3) (layers "F.Cu" "B.Cu") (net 2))
 (via (at 115.7 106.6) (size 0.6) (drill 0.3) (layers "F.Cu" "B.Cu") (free) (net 2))
 (via (at 114.8 94.3) (size 0.6) (drill 0.3) (layers "F.Cu" "B.Cu") (free) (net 2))
 (via (at 112.5 105.5) (size 0.6) (drill 0.3) (layers "F.Cu" "B.Cu") (free) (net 2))
 (via (at 120.5 102) (size 0.6) (drill 0.3) (layers "F.Cu" "B.Cu") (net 2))
 (via (at 116.5 104) (size 0.6) (drill 0.3) (layers "F.Cu" "B.Cu") (free) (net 2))
 (via (at 118.4 94.3) (size 0.6) (drill 0.3) (layers "F.Cu" "B.Cu") (free) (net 2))
 (via (at 112.5 102) (size 0.6) (drill 0.3) (layers "F.Cu" "B.Cu") (free) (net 2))
 (via (at 113.5 104.5) (size 0.6) (drill 0.3) (layers "F.Cu" "B.Cu") (free) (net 2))
 (via (at 113.2 94.3) (size 0.6) (drill 0.3) (layers "F.Cu" "B.Cu") (free) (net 2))
 (via (at 121.9 104.5) (size 0.6) (drill 0.3) (layers "F.Cu" "B.Cu") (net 2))
 (via (at 112.1 99.3) (size 0.6) (drill 0.3) (layers "F.Cu" "B.Cu") (free) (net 2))
 (via (at 118.4 105.7) (size 0.6) (drill 0.3) (layers "F.Cu" "B.Cu") (free) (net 2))
 (via (at 124.1 101.4) (size 0.6) (drill 0.3) (layers "F.Cu" "B.Cu") (free) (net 2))
 (via (at 112.1 98) (size 0.6) (drill 0.3) (layers "F.Cu" "B.Cu") (free) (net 2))
 (via (at 110.1 96) (size 0.6) (drill 0.3) (layers "F.Cu" "B.Cu") (free) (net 2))
 (via (at 118.4 100) (size 0.6) (drill 0.3) (layers "F.Cu" "B.Cu") (free) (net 2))
 (via (at 120.5 104) (size 0.6) (drill 0.3) (layers "F.Cu" "B.Cu") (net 2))
 (via (at 122.3 106.6) (size 0.6) (drill 0.3) (layers "F.Cu" "B.Cu") (free) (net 2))
 (via (at 124.1 93.4) (size 0.6) (drill 0.3) (layers "F.Cu" "B.Cu") (free) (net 2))
 (segment (start 108.4 101.25) (end 107.44 101.25) (width 0.6) (layer "F.Cu") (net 5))
 (segment (start 110.6 101.05) (end 110.6 102.975) (width 0.757) (layer "F.Cu") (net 3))
 (segment (start 110.6 102.975) (end 110.625 103) (width 0.757) (layer "F.Cu") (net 3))
 (segment (start 112.1 101.11) (end 110.66 101.11) (width 0.757) (layer "F.Cu") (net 3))
 (segment (start 110.66 101.11) (end 110.6 101.05) (width 0.757) (layer "F.Cu") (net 3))
 (segment (start 116.015 103) (end 115 103) (width 0.757) (layer "F.Cu") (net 9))
 (segment (start 113.575 103) (end 115 103) (width 0.757) (layer "F.Cu") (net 9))
 (segment (start 107.81 98) (end 107.4 98.41) (width 0.15) (layer "F.Cu") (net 6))
 (segment (start 108.39 98) (end 107.81 98) (width 0.15) (layer "F.Cu") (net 6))
 (segment (start 107.4 100.19) (end 107.4 98.41) (width 0.15) (layer "F.Cu") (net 6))
 (segment (start 116.985 103) (end 118 103) (width 0.757) (layer "F.Cu") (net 1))
 (segment (start 118 103) (end 121 103) (width 0.757) (layer "F.Cu") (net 1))
 (segment (start 121 97) (end 117.7 97) (width 0.6) (layer "F.Cu") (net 7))
 (segment (start 117.1 96.4) (end 114.6 96.4) (width 0.6) (layer "F.Cu") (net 7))
 (segment (start 117.7 97) (end 117.1 96.4) (width 0.6) (layer "F.Cu") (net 7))
 (segment (start 113.2 96.4) (end 111.55 96.4) (width 0.6) (layer "F.Cu") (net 4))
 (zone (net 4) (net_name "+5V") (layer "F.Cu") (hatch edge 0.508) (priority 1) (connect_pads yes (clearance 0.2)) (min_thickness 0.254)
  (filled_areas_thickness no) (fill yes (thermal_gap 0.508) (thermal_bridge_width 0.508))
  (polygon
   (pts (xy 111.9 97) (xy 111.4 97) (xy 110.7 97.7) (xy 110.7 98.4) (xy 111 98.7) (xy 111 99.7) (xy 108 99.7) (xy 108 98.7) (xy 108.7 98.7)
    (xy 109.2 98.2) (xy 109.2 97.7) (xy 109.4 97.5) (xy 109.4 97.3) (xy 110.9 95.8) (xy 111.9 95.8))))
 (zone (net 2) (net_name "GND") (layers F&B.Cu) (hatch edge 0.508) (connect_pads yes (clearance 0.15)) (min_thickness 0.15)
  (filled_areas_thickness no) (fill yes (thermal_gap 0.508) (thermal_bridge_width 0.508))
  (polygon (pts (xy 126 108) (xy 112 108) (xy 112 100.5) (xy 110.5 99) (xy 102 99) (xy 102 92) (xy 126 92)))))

